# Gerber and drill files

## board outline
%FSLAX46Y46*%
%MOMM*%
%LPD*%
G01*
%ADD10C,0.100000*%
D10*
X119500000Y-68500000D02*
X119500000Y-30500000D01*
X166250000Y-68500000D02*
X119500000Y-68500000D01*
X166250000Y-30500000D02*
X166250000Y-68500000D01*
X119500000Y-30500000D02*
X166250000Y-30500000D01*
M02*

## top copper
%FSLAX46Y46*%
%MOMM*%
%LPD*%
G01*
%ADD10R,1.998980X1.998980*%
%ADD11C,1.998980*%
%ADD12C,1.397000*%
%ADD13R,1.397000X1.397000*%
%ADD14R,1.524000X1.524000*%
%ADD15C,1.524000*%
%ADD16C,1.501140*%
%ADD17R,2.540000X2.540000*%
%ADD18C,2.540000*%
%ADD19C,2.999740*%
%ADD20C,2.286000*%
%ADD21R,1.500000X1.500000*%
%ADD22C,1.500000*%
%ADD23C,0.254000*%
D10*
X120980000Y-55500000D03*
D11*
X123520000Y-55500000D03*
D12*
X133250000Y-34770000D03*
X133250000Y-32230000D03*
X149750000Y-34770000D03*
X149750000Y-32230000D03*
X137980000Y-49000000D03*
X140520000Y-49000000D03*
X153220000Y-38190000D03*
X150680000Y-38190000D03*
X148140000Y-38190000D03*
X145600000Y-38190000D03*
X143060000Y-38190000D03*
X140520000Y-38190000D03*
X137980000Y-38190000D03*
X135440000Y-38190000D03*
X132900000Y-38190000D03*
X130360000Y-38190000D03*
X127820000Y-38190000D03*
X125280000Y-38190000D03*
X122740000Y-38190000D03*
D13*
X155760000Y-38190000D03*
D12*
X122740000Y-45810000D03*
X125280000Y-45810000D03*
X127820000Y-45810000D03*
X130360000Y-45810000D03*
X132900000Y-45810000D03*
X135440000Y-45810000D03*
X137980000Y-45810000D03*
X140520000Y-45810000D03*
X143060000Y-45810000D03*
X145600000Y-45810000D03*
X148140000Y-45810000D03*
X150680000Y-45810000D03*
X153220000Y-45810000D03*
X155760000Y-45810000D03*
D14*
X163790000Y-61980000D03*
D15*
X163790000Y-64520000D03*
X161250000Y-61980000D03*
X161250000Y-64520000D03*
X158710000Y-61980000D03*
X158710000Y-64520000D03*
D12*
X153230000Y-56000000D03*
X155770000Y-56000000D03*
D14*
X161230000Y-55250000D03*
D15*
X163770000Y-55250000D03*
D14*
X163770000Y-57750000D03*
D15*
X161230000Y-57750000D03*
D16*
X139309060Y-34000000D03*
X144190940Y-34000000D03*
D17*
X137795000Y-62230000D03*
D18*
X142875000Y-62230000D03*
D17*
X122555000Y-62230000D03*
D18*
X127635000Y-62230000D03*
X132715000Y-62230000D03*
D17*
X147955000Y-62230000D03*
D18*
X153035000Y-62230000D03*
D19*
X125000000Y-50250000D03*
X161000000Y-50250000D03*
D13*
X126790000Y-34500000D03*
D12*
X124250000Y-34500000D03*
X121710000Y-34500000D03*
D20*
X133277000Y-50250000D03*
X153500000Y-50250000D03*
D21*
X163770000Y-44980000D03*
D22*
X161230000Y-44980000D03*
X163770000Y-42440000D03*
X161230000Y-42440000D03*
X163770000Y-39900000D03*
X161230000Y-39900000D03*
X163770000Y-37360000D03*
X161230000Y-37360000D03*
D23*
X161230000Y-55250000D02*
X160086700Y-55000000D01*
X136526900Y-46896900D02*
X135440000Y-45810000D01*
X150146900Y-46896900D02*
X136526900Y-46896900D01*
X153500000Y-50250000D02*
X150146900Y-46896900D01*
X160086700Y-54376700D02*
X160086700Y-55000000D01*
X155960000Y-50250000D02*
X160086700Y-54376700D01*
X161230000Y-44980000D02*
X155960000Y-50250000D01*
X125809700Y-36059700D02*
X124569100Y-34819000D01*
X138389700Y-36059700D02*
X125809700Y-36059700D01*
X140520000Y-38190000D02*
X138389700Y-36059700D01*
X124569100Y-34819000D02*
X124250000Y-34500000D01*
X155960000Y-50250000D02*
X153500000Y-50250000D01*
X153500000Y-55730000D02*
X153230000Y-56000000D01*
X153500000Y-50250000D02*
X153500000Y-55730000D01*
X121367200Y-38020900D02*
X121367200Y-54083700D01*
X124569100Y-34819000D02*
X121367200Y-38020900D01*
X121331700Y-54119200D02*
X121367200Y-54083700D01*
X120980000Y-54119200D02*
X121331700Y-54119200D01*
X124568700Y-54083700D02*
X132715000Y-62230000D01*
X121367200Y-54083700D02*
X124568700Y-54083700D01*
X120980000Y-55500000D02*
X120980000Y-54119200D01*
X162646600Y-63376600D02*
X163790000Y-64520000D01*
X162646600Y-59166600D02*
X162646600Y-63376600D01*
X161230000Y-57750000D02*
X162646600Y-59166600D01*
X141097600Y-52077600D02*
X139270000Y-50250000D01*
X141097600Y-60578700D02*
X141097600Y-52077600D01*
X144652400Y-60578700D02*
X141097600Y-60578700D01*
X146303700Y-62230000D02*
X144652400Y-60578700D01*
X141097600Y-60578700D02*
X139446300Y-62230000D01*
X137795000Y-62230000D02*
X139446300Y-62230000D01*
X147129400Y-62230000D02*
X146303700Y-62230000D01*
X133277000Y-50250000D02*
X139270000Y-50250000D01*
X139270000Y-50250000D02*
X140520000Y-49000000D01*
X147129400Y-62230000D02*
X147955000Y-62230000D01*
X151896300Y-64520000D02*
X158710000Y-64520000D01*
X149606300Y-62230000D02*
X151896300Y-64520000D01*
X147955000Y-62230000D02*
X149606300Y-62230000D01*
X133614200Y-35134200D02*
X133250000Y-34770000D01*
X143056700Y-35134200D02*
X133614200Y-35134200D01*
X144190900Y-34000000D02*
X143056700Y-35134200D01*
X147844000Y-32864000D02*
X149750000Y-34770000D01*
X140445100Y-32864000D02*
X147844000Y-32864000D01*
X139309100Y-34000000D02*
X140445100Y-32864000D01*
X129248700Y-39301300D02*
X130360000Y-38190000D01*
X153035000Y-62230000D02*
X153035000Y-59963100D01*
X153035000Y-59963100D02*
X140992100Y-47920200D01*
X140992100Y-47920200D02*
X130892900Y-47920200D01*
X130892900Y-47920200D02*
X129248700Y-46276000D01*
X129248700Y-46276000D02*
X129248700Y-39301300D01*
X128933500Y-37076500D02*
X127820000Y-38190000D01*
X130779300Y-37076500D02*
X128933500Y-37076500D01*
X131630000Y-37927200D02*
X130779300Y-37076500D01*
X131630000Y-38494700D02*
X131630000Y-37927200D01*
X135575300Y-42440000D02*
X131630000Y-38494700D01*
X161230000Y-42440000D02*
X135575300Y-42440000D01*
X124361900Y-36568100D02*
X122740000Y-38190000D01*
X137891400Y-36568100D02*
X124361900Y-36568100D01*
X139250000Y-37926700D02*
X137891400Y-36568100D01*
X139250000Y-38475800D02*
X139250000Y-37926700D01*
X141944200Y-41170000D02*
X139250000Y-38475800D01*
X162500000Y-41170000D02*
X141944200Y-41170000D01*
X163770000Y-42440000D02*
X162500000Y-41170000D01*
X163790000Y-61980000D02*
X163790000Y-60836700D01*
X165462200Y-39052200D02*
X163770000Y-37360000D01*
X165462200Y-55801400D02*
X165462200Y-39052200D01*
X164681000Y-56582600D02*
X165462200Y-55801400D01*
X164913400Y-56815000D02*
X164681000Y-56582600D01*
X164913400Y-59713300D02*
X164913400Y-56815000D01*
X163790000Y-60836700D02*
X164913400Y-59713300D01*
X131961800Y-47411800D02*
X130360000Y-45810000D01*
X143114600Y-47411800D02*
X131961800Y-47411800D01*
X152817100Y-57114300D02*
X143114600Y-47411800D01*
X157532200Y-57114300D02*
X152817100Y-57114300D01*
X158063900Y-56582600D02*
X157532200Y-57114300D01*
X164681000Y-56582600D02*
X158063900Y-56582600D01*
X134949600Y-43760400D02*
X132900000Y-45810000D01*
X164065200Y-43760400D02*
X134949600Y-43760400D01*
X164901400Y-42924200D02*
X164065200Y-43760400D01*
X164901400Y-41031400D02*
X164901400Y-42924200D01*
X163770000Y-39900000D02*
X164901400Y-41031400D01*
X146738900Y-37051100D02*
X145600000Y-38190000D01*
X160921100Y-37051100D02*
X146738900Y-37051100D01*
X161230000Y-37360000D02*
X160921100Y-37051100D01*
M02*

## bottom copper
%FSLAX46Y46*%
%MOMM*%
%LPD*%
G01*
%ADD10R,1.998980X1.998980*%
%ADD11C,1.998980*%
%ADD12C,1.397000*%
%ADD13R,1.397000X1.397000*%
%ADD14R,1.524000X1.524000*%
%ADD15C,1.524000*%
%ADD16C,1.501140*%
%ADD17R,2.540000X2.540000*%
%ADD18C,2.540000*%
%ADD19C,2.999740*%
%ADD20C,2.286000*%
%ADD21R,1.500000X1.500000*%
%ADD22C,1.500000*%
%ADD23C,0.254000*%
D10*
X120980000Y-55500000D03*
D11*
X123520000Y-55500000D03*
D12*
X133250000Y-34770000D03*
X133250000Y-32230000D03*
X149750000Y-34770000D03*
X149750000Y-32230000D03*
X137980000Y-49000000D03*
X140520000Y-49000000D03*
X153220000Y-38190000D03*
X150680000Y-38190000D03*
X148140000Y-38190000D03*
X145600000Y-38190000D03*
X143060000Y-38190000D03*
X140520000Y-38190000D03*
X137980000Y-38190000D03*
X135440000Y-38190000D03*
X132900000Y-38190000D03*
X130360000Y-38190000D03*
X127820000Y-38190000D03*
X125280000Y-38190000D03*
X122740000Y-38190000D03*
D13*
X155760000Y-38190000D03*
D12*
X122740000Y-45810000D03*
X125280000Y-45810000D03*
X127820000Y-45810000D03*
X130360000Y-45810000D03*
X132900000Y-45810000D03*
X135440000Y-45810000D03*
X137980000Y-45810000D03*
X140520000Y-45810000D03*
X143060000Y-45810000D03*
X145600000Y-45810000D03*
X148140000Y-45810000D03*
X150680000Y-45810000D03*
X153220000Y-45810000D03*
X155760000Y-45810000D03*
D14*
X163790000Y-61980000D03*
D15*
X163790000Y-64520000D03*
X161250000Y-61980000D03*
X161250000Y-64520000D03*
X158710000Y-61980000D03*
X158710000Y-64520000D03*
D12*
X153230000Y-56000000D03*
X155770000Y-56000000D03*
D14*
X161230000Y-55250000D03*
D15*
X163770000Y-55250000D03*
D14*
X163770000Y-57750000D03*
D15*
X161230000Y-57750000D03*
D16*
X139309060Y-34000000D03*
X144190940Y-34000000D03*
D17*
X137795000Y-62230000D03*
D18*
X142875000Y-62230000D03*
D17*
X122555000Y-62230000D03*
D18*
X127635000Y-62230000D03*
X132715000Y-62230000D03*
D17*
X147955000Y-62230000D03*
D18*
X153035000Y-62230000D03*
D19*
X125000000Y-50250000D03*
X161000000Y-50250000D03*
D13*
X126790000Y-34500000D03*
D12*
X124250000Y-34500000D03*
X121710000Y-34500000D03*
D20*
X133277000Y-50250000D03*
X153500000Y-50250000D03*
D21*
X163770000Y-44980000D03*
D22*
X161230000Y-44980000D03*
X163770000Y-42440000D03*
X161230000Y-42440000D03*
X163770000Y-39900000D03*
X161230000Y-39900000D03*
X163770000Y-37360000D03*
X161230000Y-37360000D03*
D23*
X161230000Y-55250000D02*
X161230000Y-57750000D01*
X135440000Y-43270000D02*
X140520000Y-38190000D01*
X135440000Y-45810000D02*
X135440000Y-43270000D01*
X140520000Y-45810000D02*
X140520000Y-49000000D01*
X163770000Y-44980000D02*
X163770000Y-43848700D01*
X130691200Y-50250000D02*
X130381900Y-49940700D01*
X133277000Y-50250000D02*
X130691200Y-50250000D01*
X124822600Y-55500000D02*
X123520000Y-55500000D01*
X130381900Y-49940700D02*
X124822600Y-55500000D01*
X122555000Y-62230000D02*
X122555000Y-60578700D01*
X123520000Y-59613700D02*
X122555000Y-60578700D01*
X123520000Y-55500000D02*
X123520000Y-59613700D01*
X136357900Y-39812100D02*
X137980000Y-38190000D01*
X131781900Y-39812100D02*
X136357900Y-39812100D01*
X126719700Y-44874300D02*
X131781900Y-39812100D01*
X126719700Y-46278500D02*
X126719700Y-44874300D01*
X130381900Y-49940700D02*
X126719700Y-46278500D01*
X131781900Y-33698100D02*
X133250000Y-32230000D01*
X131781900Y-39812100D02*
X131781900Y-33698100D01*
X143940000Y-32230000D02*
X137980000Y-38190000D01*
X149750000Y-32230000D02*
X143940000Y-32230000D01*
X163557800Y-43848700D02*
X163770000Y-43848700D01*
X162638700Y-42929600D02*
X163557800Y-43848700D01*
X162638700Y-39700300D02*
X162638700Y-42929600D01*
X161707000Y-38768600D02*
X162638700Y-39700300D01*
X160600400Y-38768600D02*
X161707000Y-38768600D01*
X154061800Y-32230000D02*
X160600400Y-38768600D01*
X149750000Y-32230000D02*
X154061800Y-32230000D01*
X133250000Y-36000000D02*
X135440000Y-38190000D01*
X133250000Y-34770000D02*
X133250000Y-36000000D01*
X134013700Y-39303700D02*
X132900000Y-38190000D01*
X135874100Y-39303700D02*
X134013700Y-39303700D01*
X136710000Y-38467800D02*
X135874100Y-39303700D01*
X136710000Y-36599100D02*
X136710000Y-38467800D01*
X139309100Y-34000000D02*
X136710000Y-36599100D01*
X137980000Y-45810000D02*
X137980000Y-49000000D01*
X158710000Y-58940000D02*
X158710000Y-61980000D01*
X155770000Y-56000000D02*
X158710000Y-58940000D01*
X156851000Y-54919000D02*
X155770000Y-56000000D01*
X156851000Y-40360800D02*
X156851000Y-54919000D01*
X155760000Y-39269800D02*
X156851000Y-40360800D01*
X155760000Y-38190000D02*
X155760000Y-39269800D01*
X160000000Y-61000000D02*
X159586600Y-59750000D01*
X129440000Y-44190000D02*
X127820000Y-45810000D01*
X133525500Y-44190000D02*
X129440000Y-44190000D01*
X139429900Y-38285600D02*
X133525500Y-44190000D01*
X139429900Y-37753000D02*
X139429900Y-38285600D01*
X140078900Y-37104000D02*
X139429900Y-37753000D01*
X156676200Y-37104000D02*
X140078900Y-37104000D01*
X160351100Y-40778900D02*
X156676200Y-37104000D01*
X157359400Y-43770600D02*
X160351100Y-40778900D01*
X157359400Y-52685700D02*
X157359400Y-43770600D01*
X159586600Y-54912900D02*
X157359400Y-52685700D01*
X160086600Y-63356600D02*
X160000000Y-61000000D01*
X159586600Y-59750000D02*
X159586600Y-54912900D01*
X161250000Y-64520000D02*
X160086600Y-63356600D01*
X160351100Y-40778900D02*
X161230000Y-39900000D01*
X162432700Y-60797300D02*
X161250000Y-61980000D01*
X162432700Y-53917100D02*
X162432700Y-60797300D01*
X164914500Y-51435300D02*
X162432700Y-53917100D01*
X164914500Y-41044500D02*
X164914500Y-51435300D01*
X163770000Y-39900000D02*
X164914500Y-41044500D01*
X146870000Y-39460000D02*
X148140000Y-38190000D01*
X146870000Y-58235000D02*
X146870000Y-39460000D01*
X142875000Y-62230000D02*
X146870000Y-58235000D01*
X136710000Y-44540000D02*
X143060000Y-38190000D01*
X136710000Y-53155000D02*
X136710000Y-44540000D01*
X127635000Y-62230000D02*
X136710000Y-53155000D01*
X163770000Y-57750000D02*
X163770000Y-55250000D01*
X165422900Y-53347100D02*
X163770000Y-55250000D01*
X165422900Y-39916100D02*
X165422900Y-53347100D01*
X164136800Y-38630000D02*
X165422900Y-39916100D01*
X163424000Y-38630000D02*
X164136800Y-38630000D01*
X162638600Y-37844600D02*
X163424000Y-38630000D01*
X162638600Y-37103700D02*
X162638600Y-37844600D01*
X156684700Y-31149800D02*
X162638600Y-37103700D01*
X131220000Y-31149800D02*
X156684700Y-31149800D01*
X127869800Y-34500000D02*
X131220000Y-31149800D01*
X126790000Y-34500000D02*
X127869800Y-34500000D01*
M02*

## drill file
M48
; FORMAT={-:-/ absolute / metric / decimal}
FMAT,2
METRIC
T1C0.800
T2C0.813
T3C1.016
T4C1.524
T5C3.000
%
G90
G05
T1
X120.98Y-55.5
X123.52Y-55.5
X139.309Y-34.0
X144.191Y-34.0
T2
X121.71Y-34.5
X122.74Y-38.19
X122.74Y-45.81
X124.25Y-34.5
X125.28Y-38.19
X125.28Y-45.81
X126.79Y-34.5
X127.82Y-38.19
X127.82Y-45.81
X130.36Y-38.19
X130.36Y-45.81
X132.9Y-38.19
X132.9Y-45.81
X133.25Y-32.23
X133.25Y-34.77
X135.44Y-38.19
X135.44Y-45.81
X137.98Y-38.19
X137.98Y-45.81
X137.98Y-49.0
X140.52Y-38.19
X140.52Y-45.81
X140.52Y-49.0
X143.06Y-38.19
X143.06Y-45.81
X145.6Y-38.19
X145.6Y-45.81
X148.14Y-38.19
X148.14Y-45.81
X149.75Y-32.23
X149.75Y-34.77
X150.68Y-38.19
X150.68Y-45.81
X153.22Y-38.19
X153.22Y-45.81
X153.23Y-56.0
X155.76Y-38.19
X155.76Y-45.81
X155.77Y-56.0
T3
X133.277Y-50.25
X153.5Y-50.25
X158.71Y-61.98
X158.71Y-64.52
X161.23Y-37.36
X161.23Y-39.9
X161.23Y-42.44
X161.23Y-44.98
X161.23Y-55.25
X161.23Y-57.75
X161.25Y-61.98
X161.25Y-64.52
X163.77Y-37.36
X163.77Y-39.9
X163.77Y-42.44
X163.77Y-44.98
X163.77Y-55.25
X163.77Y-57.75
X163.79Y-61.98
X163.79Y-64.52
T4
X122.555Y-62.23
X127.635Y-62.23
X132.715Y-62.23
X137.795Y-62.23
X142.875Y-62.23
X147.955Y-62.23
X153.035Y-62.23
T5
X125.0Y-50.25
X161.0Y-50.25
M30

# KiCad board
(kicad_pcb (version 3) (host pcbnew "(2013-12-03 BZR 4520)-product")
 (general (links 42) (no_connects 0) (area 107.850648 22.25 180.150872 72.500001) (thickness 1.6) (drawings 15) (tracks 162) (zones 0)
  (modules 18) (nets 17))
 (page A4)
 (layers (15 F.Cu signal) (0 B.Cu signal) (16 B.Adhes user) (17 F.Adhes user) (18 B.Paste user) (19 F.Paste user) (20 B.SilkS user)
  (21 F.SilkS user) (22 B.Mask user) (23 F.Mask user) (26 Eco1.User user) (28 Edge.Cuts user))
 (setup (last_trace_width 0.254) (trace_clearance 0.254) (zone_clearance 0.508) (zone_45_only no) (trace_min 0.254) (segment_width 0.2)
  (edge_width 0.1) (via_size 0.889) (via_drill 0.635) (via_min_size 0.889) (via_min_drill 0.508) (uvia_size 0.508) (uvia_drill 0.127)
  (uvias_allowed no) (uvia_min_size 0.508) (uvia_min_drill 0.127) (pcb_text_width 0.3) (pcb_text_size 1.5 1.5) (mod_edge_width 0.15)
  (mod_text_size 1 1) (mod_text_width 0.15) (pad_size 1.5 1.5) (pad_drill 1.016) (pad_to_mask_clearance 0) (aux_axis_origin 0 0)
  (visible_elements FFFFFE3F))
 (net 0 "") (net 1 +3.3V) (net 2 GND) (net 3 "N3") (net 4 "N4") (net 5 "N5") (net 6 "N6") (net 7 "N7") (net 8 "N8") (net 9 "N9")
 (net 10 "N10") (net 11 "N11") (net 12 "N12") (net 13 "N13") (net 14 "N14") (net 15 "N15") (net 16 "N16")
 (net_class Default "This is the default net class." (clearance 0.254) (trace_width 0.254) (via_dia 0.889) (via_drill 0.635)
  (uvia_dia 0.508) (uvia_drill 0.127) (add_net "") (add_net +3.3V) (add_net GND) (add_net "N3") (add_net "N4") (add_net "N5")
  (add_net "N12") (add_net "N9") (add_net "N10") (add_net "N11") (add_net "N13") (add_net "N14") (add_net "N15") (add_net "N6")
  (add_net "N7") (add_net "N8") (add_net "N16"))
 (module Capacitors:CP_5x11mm (layer F.Cu) (at 122.25 55.5 270)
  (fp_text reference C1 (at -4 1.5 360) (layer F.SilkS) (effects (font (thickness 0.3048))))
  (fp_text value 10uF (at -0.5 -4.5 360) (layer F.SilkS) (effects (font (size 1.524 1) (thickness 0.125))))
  (pad 1 thru_hole rect (at 0 1.27 270) (size 1.99898 1.99898) (drill 0.8001) (layers *.Cu *.Mask F.SilkS) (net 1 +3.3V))
  (pad 2 thru_hole circle (at 0 -1.27 270) (size 1.99898 1.99898) (drill 0.8001) (layers *.Cu *.Mask F.SilkS) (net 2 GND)))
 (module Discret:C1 (layer F.Cu) (at 133.25 33.5 90)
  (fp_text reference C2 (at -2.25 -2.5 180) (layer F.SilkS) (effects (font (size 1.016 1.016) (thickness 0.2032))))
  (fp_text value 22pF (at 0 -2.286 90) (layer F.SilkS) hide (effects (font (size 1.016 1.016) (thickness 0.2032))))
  (pad 1 thru_hole circle (at -1.27 0 90) (size 1.397 1.397) (drill 0.8128) (layers *.Cu *.Mask F.SilkS) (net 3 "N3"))
  (pad 2 thru_hole circle (at 1.27 0 90) (size 1.397 1.397) (drill 0.8128) (layers *.Cu *.Mask F.SilkS) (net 2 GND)))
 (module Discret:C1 (layer F.Cu) (at 149.75 33.5 90)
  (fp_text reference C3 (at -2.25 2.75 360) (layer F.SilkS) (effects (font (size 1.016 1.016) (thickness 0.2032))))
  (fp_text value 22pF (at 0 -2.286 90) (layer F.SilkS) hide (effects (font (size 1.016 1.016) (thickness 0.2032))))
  (pad 1 thru_hole circle (at -1.27 0 90) (size 1.397 1.397) (drill 0.8128) (layers *.Cu *.Mask F.SilkS) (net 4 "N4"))
  (pad 2 thru_hole circle (at 1.27 0 90) (size 1.397 1.397) (drill 0.8128) (layers *.Cu *.Mask F.SilkS) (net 2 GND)))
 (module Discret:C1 (layer F.Cu) (at 139.25 49)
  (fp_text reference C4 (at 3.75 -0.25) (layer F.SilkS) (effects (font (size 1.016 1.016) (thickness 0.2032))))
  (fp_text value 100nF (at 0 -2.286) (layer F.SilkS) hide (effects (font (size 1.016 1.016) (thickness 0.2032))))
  (pad 1 thru_hole circle (at -1.27 0) (size 1.397 1.397) (drill 0.8128) (layers *.Cu *.Mask F.SilkS) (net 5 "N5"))
  (pad 2 thru_hole circle (at 1.27 0) (size 1.397 1.397) (drill 0.8128) (layers *.Cu *.Mask F.SilkS) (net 2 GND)))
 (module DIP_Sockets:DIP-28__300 (layer F.Cu) (at 139.25 42 180)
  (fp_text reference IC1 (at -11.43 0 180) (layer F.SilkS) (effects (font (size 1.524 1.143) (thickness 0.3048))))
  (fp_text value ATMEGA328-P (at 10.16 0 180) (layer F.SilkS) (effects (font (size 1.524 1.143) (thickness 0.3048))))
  (pad 2 thru_hole circle (at -13.97 3.81 180) (size 1.397 1.397) (drill 0.8128) (layers *.Cu *.Mask F.SilkS))
  (pad 3 thru_hole circle (at -11.43 3.81 180) (size 1.397 1.397) (drill 0.8128) (layers *.Cu *.Mask F.SilkS))
  (pad 4 thru_hole circle (at -8.89 3.81 180) (size 1.397 1.397) (drill 0.8128) (layers *.Cu *.Mask F.SilkS) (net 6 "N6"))
  (pad 5 thru_hole circle (at -6.35 3.81 180) (size 1.397 1.397) (drill 0.8128) (layers *.Cu *.Mask F.SilkS) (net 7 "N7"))
  (pad 6 thru_hole circle (at -3.81 3.81 180) (size 1.397 1.397) (drill 0.8128) (layers *.Cu *.Mask F.SilkS) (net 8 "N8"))
  (pad 7 thru_hole circle (at -1.27 3.81 180) (size 1.397 1.397) (drill 0.8128) (layers *.Cu *.Mask F.SilkS) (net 1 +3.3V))
  (pad 8 thru_hole circle (at 1.27 3.81 180) (size 1.397 1.397) (drill 0.8128) (layers *.Cu *.Mask F.SilkS) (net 2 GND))
  (pad 9 thru_hole circle (at 3.81 3.81 180) (size 1.397 1.397) (drill 0.8128) (layers *.Cu *.Mask F.SilkS) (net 3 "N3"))
  (pad 10 thru_hole circle (at 6.35 3.81 180) (size 1.397 1.397) (drill 0.8128) (layers *.Cu *.Mask F.SilkS) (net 4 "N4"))
  (pad 11 thru_hole circle (at 8.89 3.81 180) (size 1.397 1.397) (drill 0.8128) (layers *.Cu *.Mask F.SilkS) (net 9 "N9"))
  (pad 12 thru_hole circle (at 11.43 3.81 180) (size 1.397 1.397) (drill 0.8128) (layers *.Cu *.Mask F.SilkS) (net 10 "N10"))
  (pad 13 thru_hole circle (at 13.97 3.81 180) (size 1.397 1.397) (drill 0.8128) (layers *.Cu *.Mask F.SilkS))
  (pad 14 thru_hole circle (at 16.51 3.81 180) (size 1.397 1.397) (drill 0.8128) (layers *.Cu *.Mask F.SilkS) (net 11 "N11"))
  (pad 1 thru_hole rect (at -16.51 3.81 180) (size 1.397 1.397) (drill 0.8128) (layers *.Cu *.Mask F.SilkS) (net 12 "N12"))
  (pad 15 thru_hole circle (at 16.51 -3.81 180) (size 1.397 1.397) (drill 0.8128) (layers *.Cu *.Mask F.SilkS))
  (pad 16 thru_hole circle (at 13.97 -3.81 180) (size 1.397 1.397) (drill 0.8128) (layers *.Cu *.Mask F.SilkS))
  (pad 17 thru_hole circle (at 11.43 -3.81 180) (size 1.397 1.397) (drill 0.8128) (layers *.Cu *.Mask F.SilkS) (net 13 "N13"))
  (pad 18 thru_hole circle (at 8.89 -3.81 180) (size 1.397 1.397) (drill 0.8128) (layers *.Cu *.Mask F.SilkS) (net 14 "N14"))
  (pad 19 thru_hole circle (at 6.35 -3.81 180) (size 1.397 1.397) (drill 0.8128) (layers *.Cu *.Mask F.SilkS) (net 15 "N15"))
  (pad 20 thru_hole circle (at 3.81 -3.81 180) (size 1.397 1.397) (drill 0.8128) (layers *.Cu *.Mask F.SilkS) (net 1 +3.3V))
  (pad 21 thru_hole circle (at 1.27 -3.81 180) (size 1.397 1.397) (drill 0.8128) (layers *.Cu *.Mask F.SilkS) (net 5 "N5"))
  (pad 22 thru_hole circle (at -1.27 -3.81 180) (size 1.397 1.397) (drill 0.8128) (layers *.Cu *.Mask F.SilkS) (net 2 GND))
  (pad 23 thru_hole circle (at -3.81 -3.81 180) (size 1.397 1.397) (drill 0.8128) (layers *.Cu *.Mask F.SilkS))
  (pad 24 thru_hole circle (at -6.35 -3.81 180) (size 1.397 1.397) (drill 0.8128) (layers *.Cu *.Mask F.SilkS))
  (pad 25 thru_hole circle (at -8.89 -3.81 180) (size 1.397 1.397) (drill 0.8128) (layers *.Cu *.Mask F.SilkS))
  (pad 26 thru_hole circle (at -11.43 -3.81 180) (size 1.397 1.397) (drill 0.8128) (layers *.Cu *.Mask F.SilkS))
  (pad 27 thru_hole circle (at -13.97 -3.81 180) (size 1.397 1.397) (drill 0.8128) (layers *.Cu *.Mask F.SilkS))
  (pad 28 thru_hole circle (at -16.51 -3.81 180) (size 1.397 1.397) (drill 0.8128) (layers *.Cu *.Mask F.SilkS)))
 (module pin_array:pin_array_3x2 (layer F.Cu) (at 161.25 63.25 180)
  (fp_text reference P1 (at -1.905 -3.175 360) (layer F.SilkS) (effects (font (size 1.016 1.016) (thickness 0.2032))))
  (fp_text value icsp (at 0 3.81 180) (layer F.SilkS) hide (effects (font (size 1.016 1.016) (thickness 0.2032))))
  (pad 1 thru_hole rect (at -2.54 1.27 180) (size 1.524 1.524) (drill 1.016) (layers *.Cu *.Mask F.SilkS) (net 14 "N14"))
  (pad 2 thru_hole circle (at -2.54 -1.27 180) (size 1.524 1.524) (drill 1.016) (layers *.Cu *.Mask F.SilkS) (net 1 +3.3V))
  (pad 3 thru_hole circle (at 0 1.27 180) (size 1.524 1.524) (drill 1.016) (layers *.Cu *.Mask F.SilkS) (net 15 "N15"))
  (pad 4 thru_hole circle (at 0 -1.27 180) (size 1.524 1.524) (drill 1.016) (layers *.Cu *.Mask F.SilkS) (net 13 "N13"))
  (pad 5 thru_hole circle (at 2.54 1.27 180) (size 1.524 1.524) (drill 1.016) (layers *.Cu *.Mask F.SilkS) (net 12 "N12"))
  (pad 6 thru_hole circle (at 2.54 -1.27 180) (size 1.524 1.524) (drill 1.016) (layers *.Cu *.Mask F.SilkS) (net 2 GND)))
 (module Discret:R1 (layer F.Cu) (at 154.5 56) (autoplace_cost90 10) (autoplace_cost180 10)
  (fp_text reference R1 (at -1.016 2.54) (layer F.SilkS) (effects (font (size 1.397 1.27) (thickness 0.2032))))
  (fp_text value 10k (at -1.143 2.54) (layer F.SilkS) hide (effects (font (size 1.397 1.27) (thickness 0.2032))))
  (pad 1 thru_hole circle (at -1.27 0) (size 1.397 1.397) (drill 0.8128) (layers *.Cu *.Mask F.SilkS) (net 1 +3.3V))
  (pad 2 thru_hole circle (at 1.27 0) (size 1.397 1.397) (drill 0.8128) (layers *.Cu *.Mask F.SilkS) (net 12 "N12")))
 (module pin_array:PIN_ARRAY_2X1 (layer F.Cu) (at 162.5 55.25)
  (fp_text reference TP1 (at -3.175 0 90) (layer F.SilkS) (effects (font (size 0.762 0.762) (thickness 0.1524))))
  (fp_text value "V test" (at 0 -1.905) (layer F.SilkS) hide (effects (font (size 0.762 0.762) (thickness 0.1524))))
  (pad 1 thru_hole rect (at -1.27 0) (size 1.524 1.524) (drill 1.016) (layers *.Cu *.Mask F.SilkS) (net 1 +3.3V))
  (pad 2 thru_hole circle (at 1.27 0) (size 1.524 1.524) (drill 1.016) (layers *.Cu *.Mask F.SilkS) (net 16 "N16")))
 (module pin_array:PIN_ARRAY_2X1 (layer F.Cu) (at 162.5 57.75 180)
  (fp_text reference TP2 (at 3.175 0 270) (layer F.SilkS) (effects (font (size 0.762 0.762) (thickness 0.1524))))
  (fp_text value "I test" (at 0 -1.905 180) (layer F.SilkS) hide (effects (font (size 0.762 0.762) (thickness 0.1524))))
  (pad 1 thru_hole rect (at -1.27 0 180) (size 1.524 1.524) (drill 1.016) (layers *.Cu *.Mask F.SilkS) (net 16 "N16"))
  (pad 2 thru_hole circle (at 1.27 0 180) (size 1.524 1.524) (drill 1.016) (layers *.Cu *.Mask F.SilkS) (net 1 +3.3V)))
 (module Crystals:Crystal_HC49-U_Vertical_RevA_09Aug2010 (layer F.Cu) (at 141.75 34)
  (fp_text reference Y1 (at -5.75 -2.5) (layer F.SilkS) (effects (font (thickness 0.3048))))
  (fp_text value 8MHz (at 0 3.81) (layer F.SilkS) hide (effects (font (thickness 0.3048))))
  (pad 1 thru_hole circle (at -2.44094 0) (size 1.50114 1.50114) (drill 0.8001) (layers *.Cu *.Mask F.SilkS) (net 4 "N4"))
  (pad 2 thru_hole circle (at 2.44094 0) (size 1.50114 1.50114) (drill 0.8001) (layers *.Cu *.Mask F.SilkS) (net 3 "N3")))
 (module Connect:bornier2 (layer F.Cu) (at 140.335 62.23)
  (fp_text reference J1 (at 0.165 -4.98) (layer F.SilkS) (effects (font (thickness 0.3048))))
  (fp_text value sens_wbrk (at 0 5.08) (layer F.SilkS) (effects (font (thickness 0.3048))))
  (pad 1 thru_hole rect (at -2.54 0) (size 2.54 2.54) (drill 1.524) (layers *.Cu *.Mask F.SilkS) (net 2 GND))
  (pad 2 thru_hole circle (at 2.54 0) (size 2.54 2.54) (drill 1.524) (layers *.Cu *.Mask F.SilkS) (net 6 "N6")))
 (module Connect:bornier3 (layer F.Cu) (at 127.635 62.23)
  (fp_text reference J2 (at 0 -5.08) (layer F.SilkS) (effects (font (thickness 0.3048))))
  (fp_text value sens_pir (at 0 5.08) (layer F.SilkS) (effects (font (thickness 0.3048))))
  (pad 1 thru_hole rect (at -5.08 0) (size 2.54 2.54) (drill 1.524) (layers *.Cu *.Mask F.SilkS) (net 2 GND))
  (pad 2 thru_hole circle (at 0 0) (size 2.54 2.54) (drill 1.524) (layers *.Cu *.Mask F.SilkS) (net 8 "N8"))
  (pad 3 thru_hole circle (at 5.08 0) (size 2.54 2.54) (drill 1.524) (layers *.Cu *.Mask F.SilkS) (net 1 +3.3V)))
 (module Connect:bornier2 (layer F.Cu) (at 150.495 62.23)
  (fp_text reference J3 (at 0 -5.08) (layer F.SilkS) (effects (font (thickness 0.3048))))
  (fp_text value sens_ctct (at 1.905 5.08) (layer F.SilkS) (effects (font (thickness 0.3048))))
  (pad 1 thru_hole rect (at -2.54 0) (size 2.54 2.54) (drill 1.524) (layers *.Cu *.Mask F.SilkS) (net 2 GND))
  (pad 2 thru_hole circle (at 2.54 0) (size 2.54 2.54) (drill 1.524) (layers *.Cu *.Mask F.SilkS) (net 9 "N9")))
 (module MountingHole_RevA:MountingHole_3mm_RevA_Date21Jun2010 (layer F.Cu) (at 125 50.25) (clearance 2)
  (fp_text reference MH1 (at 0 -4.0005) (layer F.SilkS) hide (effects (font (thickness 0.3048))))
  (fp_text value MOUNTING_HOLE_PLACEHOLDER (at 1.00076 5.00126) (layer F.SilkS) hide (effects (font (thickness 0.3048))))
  (pad 1 thru_hole circle (at 0 0) (size 2.99974 2.99974) (drill 2.99974) (layers)))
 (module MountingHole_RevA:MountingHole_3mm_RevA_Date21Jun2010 (layer F.Cu) (at 161 50.25) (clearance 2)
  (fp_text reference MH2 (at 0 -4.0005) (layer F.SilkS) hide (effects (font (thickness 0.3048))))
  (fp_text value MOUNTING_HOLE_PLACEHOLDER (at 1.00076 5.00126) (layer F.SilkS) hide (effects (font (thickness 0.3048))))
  (pad 1 thru_hole circle (at 0 0) (size 2.99974 2.99974) (drill 2.99974) (layers)))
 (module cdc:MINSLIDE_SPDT (layer F.Cu) (at 124.25 34.5 180)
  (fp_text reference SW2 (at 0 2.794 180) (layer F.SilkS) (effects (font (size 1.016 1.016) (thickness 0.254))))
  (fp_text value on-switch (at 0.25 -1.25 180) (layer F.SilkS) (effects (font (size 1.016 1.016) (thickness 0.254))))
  (pad 1 thru_hole rect (at -2.54 0 180) (size 1.397 1.397) (drill 0.8128) (layers *.Cu *.Mask F.SilkS) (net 16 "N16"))
  (pad 2 thru_hole circle (at 0 0 180) (size 1.397 1.397) (drill 0.8128) (layers *.Cu *.Mask F.SilkS) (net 1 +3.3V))
  (pad 3 thru_hole circle (at 2.54 0 180) (size 1.397 1.397) (drill 0.8128) (layers *.Cu *.Mask F.SilkS)))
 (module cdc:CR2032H (layer B.Cu) (at 139.5 50.25)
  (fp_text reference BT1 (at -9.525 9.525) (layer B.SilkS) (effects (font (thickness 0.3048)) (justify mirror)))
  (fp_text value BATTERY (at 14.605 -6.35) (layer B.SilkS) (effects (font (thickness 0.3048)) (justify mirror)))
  (pad 2 thru_hole circle (at -6.223 0) (size 2.286 2.286) (drill 1.016) (layers *.Cu *.Mask B.SilkS) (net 2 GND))
  (pad 1 thru_hole circle (at 14 0) (size 2.286 2.286) (drill 1.016) (layers *.Cu *.Mask B.SilkS) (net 1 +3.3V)))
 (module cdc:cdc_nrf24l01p (layer F.Cu) (at 162.5 46.25 180)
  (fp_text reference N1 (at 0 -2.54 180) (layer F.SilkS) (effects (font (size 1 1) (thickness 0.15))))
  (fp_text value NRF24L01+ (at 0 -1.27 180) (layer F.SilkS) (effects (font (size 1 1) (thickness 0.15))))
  (pad 1 thru_hole rect (at -1.27 1.27 180) (size 1.5 1.5) (drill 1.016) (layers *.Cu *.Mask F.SilkS) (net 2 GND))
  (pad 2 thru_hole circle (at 1.27 1.27 180) (size 1.5 1.5) (drill 1.016) (layers *.Cu *.Mask F.SilkS) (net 1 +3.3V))
  (pad 3 thru_hole circle (at -1.27 3.81 180) (size 1.5 1.5) (drill 1.016) (layers *.Cu *.Mask F.SilkS) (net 11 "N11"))
  (pad 4 thru_hole circle (at 1.27 3.81 180) (size 1.5 1.5) (drill 1.016) (layers *.Cu *.Mask F.SilkS) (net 10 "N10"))
  (pad 5 thru_hole circle (at -1.27 6.35 180) (size 1.5 1.5) (drill 1.016) (layers *.Cu *.Mask F.SilkS) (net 15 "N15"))
  (pad 6 thru_hole circle (at 1.27 6.35 180) (size 1.5 1.5) (drill 1.016) (layers *.Cu *.Mask F.SilkS) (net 13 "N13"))
  (pad 7 thru_hole circle (at -1.27 8.89 180) (size 1.5 1.5) (drill 1.016) (layers *.Cu *.Mask F.SilkS) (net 14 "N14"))
  (pad 8 thru_hole circle (at 1.27 8.89 180) (size 1.5 1.5) (drill 1.016) (layers *.Cu *.Mask F.SilkS) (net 7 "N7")))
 (gr_line (start 119.5 68.5) (end 119.5 30.5) (angle 90) (layer Edge.Cuts) (width 0.1))
 (gr_line (start 166.25 68.5) (end 119.5 68.5) (angle 90) (layer Edge.Cuts) (width 0.1))
 (gr_line (start 166.25 30.5) (end 166.25 68.5) (angle 90) (layer Edge.Cuts) (width 0.1))
 (gr_line (start 119.5 30.5) (end 166.25 30.5) (angle 90) (layer Edge.Cuts) (width 0.1))
 (segment (start 161.23 55.25) (end 161.23 57.75) (width 0.254) (layer B.Cu) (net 1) (status 20))
 (segment (start 161.23 55.25) (end 160.0867 55) (width 0.254) (layer F.Cu) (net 1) (status 10))
 (segment (start 136.5269 46.8969) (end 135.44 45.81) (width 0.254) (layer F.Cu) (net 1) (status 20))
 (segment (start 150.1469 46.8969) (end 136.5269 46.8969) (width 0.254) (layer F.Cu) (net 1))
 (segment (start 153.5 50.25) (end 150.1469 46.8969) (width 0.254) (layer F.Cu) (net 1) (status 10))
 (segment (start 160.0867 54.3767) (end 160.0867 55) (width 0.254) (layer F.Cu) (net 1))
 (segment (start 155.96 50.25) (end 160.0867 54.3767) (width 0.254) (layer F.Cu) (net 1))
 (segment (start 161.23 44.98) (end 155.96 50.25) (width 0.254) (layer F.Cu) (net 1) (status 10))
 (segment (start 135.44 43.27) (end 140.52 38.19) (width 0.254) (layer B.Cu) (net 1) (status 20))
 (segment (start 135.44 45.81) (end 135.44 43.27) (width 0.254) (layer B.Cu) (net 1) (status 10))
 (segment (start 125.8097 36.0597) (end 124.5691 34.819) (width 0.254) (layer F.Cu) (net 1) (status 20))
 (segment (start 138.3897 36.0597) (end 125.8097 36.0597) (width 0.254) (layer F.Cu) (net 1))
 (segment (start 140.52 38.19) (end 138.3897 36.0597) (width 0.254) (layer F.Cu) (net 1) (status 10))
 (segment (start 124.5691 34.819) (end 124.25 34.5) (width 0.254) (layer F.Cu) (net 1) (status 30))
 (segment (start 155.96 50.25) (end 153.5 50.25) (width 0.254) (layer F.Cu) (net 1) (status 20))
 (segment (start 153.5 55.73) (end 153.23 56) (width 0.254) (layer F.Cu) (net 1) (status 30))
 (segment (start 153.5 50.25) (end 153.5 55.73) (width 0.254) (layer F.Cu) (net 1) (status 30))
 (segment (start 121.3672 38.0209) (end 121.3672 54.0837) (width 0.254) (layer F.Cu) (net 1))
 (segment (start 124.5691 34.819) (end 121.3672 38.0209) (width 0.254) (layer F.Cu) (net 1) (status 10))
 (segment (start 121.3317 54.1192) (end 121.3672 54.0837) (width 0.254) (layer F.Cu) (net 1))
 (segment (start 120.98 54.1192) (end 121.3317 54.1192) (width 0.254) (layer F.Cu) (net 1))
 (segment (start 124.5687 54.0837) (end 132.715 62.23) (width 0.254) (layer F.Cu) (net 1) (status 20))
 (segment (start 121.3672 54.0837) (end 124.5687 54.0837) (width 0.254) (layer F.Cu) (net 1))
 (segment (start 120.98 55.5) (end 120.98 54.1192) (width 0.254) (layer F.Cu) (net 1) (status 10))
 (segment (start 162.6466 63.3766) (end 163.79 64.52) (width 0.254) (layer F.Cu) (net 1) (status 20))
 (segment (start 162.6466 59.1666) (end 162.6466 63.3766) (width 0.254) (layer F.Cu) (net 1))
 (segment (start 161.23 57.75) (end 162.6466 59.1666) (width 0.254) (layer F.Cu) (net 1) (status 10))
 (segment (start 141.0976 52.0776) (end 139.27 50.25) (width 0.254) (layer F.Cu) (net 2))
 (segment (start 141.0976 60.5787) (end 141.0976 52.0776) (width 0.254) (layer F.Cu) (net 2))
 (segment (start 144.6524 60.5787) (end 141.0976 60.5787) (width 0.254) (layer F.Cu) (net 2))
 (segment (start 146.3037 62.23) (end 144.6524 60.5787) (width 0.254) (layer F.Cu) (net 2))
 (segment (start 141.0976 60.5787) (end 139.4463 62.23) (width 0.254) (layer F.Cu) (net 2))
 (segment (start 140.52 45.81) (end 140.52 49) (width 0.254) (layer B.Cu) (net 2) (status 30))
 (segment (start 163.77 44.98) (end 163.77 43.8487) (width 0.254) (layer B.Cu) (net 2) (status 10))
 (segment (start 137.795 62.23) (end 139.4463 62.23) (width 0.254) (layer F.Cu) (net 2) (status 10))
 (segment (start 147.1294 62.23) (end 146.3037 62.23) (width 0.254) (layer F.Cu) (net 2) (status 10))
 (segment (start 133.277 50.25) (end 139.27 50.25) (width 0.254) (layer F.Cu) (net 2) (status 10))
 (segment (start 139.27 50.25) (end 140.52 49) (width 0.254) (layer F.Cu) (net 2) (status 20))
 (segment (start 130.6912 50.25) (end 130.3819 49.9407) (width 0.254) (layer B.Cu) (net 2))
 (segment (start 133.277 50.25) (end 130.6912 50.25) (width 0.254) (layer B.Cu) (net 2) (status 10))
 (segment (start 147.1294 62.23) (end 147.955 62.23) (width 0.254) (layer F.Cu) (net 2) (status 30))
 (segment (start 151.8963 64.52) (end 158.71 64.52) (width 0.254) (layer F.Cu) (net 2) (status 20))
 (segment (start 149.6063 62.23) (end 151.8963 64.52) (width 0.254) (layer F.Cu) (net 2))
 (segment (start 147.955 62.23) (end 149.6063 62.23) (width 0.254) (layer F.Cu) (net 2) (status 10))
 (segment (start 124.8226 55.5) (end 123.52 55.5) (width 0.254) (layer B.Cu) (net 2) (status 20))
 (segment (start 130.3819 49.9407) (end 124.8226 55.5) (width 0.254) (layer B.Cu) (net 2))
 (segment (start 122.555 62.23) (end 122.555 60.5787) (width 0.254) (layer B.Cu) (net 2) (status 10))
 (segment (start 123.52 59.6137) (end 122.555 60.5787) (width 0.254) (layer B.Cu) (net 2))
 (segment (start 123.52 55.5) (end 123.52 59.6137) (width 0.254) (layer B.Cu) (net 2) (status 10))
 (segment (start 136.3579 39.8121) (end 137.98 38.19) (width 0.254) (layer B.Cu) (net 2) (status 20))
 (segment (start 131.7819 39.8121) (end 136.3579 39.8121) (width 0.254) (layer B.Cu) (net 2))
 (segment (start 126.7197 44.8743) (end 131.7819 39.8121) (width 0.254) (layer B.Cu) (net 2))
 (segment (start 126.7197 46.2785) (end 126.7197 44.8743) (width 0.254) (layer B.Cu) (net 2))
 (segment (start 130.3819 49.9407) (end 126.7197 46.2785) (width 0.254) (layer B.Cu) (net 2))
 (segment (start 131.7819 33.6981) (end 133.25 32.23) (width 0.254) (layer B.Cu) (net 2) (status 20))
 (segment (start 131.7819 39.8121) (end 131.7819 33.6981) (width 0.254) (layer B.Cu) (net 2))
 (segment (start 143.94 32.23) (end 137.98 38.19) (width 0.254) (layer B.Cu) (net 2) (status 20))
 (segment (start 149.75 32.23) (end 143.94 32.23) (width 0.254) (layer B.Cu) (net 2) (status 10))
 (segment (start 163.5578 43.8487) (end 163.77 43.8487) (width 0.254) (layer B.Cu) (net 2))
 (segment (start 162.6387 42.9296) (end 163.5578 43.8487) (width 0.254) (layer B.Cu) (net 2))
 (segment (start 162.6387 39.7003) (end 162.6387 42.9296) (width 0.254) (layer B.Cu) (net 2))
 (segment (start 161.707 38.7686) (end 162.6387 39.7003) (width 0.254) (layer B.Cu) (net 2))
 (segment (start 160.6004 38.7686) (end 161.707 38.7686) (width 0.254) (layer B.Cu) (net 2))
 (segment (start 154.0618 32.23) (end 160.6004 38.7686) (width 0.254) (layer B.Cu) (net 2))
 (segment (start 149.75 32.23) (end 154.0618 32.23) (width 0.254) (layer B.Cu) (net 2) (status 10))
 (segment (start 133.6142 35.1342) (end 133.25 34.77) (width 0.254) (layer F.Cu) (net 3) (status 30))
 (segment (start 143.0567 35.1342) (end 133.6142 35.1342) (width 0.254) (layer F.Cu) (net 3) (status 20))
 (segment (start 144.1909 34) (end 143.0567 35.1342) (width 0.254) (layer F.Cu) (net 3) (status 10))
 (segment (start 133.25 36) (end 135.44 38.19) (width 0.254) (layer B.Cu) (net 3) (status 20))
 (segment (start 133.25 34.77) (end 133.25 36) (width 0.254) (layer B.Cu) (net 3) (status 10))
 (segment (start 147.844 32.864) (end 149.75 34.77) (width 0.254) (layer F.Cu) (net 4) (status 20))
 (segment (start 140.4451 32.864) (end 147.844 32.864) (width 0.254) (layer F.Cu) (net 4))
 (segment (start 139.3091 34) (end 140.4451 32.864) (width 0.254) (layer F.Cu) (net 4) (status 10))
 (segment (start 134.0137 39.3037) (end 132.9 38.19) (width 0.254) (layer B.Cu) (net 4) (status 20))
 (segment (start 135.8741 39.3037) (end 134.0137 39.3037) (width 0.254) (layer B.Cu) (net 4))
 (segment (start 136.71 38.4678) (end 135.8741 39.3037) (width 0.254) (layer B.Cu) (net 4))
 (segment (start 136.71 36.5991) (end 136.71 38.4678) (width 0.254) (layer B.Cu) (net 4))
 (segment (start 139.3091 34) (end 136.71 36.5991) (width 0.254) (layer B.Cu) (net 4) (status 10))
 (segment (start 137.98 45.81) (end 137.98 49) (width 0.254) (layer B.Cu) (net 5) (status 30))
 (segment (start 158.71 58.94) (end 158.71 61.98) (width 0.254) (layer B.Cu) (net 12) (status 20))
 (segment (start 155.77 56) (end 158.71 58.94) (width 0.254) (layer B.Cu) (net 12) (status 10))
 (segment (start 156.851 54.919) (end 155.77 56) (width 0.254) (layer B.Cu) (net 12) (status 20))
 (segment (start 156.851 40.3608) (end 156.851 54.919) (width 0.254) (layer B.Cu) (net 12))
 (segment (start 155.76 39.2698) (end 156.851 40.3608) (width 0.254) (layer B.Cu) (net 12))
 (segment (start 155.76 38.19) (end 155.76 39.2698) (width 0.254) (layer B.Cu) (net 12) (status 10))
 (segment (start 129.2487 39.3013) (end 130.36 38.19) (width 0.254) (layer F.Cu) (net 9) (status 20))
 (segment (start 153.035 62.23) (end 153.035 59.9631) (width 0.254) (layer F.Cu) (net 9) (status 10))
 (segment (start 153.035 59.9631) (end 140.9921 47.9202) (width 0.254) (layer F.Cu) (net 9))
 (segment (start 140.9921 47.9202) (end 130.8929 47.9202) (width 0.254) (layer F.Cu) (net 9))
 (segment (start 130.8929 47.9202) (end 129.2487 46.276) (width 0.254) (layer F.Cu) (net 9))
 (segment (start 129.2487 46.276) (end 129.2487 39.3013) (width 0.254) (layer F.Cu) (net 9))
 (segment (start 128.9335 37.0765) (end 127.82 38.19) (width 0.254) (layer F.Cu) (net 10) (status 20))
 (segment (start 130.7793 37.0765) (end 128.9335 37.0765) (width 0.254) (layer F.Cu) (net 10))
 (segment (start 131.63 37.9272) (end 130.7793 37.0765) (width 0.254) (layer F.Cu) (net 10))
 (segment (start 131.63 38.4947) (end 131.63 37.9272) (width 0.254) (layer F.Cu) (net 10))
 (segment (start 135.5753 42.44) (end 131.63 38.4947) (width 0.254) (layer F.Cu) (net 10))
 (segment (start 161.23 42.44) (end 135.5753 42.44) (width 0.254) (layer F.Cu) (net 10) (status 10))
 (segment (start 124.3619 36.5681) (end 122.74 38.19) (width 0.254) (layer F.Cu) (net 11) (status 20))
 (segment (start 137.8914 36.5681) (end 124.3619 36.5681) (width 0.254) (layer F.Cu) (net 11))
 (segment (start 139.25 37.9267) (end 137.8914 36.5681) (width 0.254) (layer F.Cu) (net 11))
 (segment (start 139.25 38.4758) (end 139.25 37.9267) (width 0.254) (layer F.Cu) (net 11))
 (segment (start 141.9442 41.17) (end 139.25 38.4758) (width 0.254) (layer F.Cu) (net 11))
 (segment (start 162.5 41.17) (end 141.9442 41.17) (width 0.254) (layer F.Cu) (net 11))
 (segment (start 163.77 42.44) (end 162.5 41.17) (width 0.254) (layer F.Cu) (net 11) (status 10))
 (segment (start 160 61) (end 159.5866 59.75) (width 0.254) (layer B.Cu) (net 13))
 (segment (start 129.44 44.19) (end 127.82 45.81) (width 0.254) (layer B.Cu) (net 13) (status 20))
 (segment (start 133.5255 44.19) (end 129.44 44.19) (width 0.254) (layer B.Cu) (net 13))
 (segment (start 139.4299 38.2856) (end 133.5255 44.19) (width 0.254) (layer B.Cu) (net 13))
 (segment (start 139.4299 37.753) (end 139.4299 38.2856) (width 0.254) (layer B.Cu) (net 13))
 (segment (start 140.0789 37.104) (end 139.4299 37.753) (width 0.254) (layer B.Cu) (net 13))
 (segment (start 156.6762 37.104) (end 140.0789 37.104) (width 0.254) (layer B.Cu) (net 13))
 (segment (start 160.3511 40.7789) (end 156.6762 37.104) (width 0.254) (layer B.Cu) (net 13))
 (segment (start 157.3594 43.7706) (end 160.3511 40.7789) (width 0.254) (layer B.Cu) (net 13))
 (segment (start 157.3594 52.6857) (end 157.3594 43.7706) (width 0.254) (layer B.Cu) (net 13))
 (segment (start 159.5866 54.9129) (end 157.3594 52.6857) (width 0.254) (layer B.Cu) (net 13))
 (segment (start 160.0866 63.3566) (end 160 61) (width 0.254) (layer B.Cu) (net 13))
 (segment (start 159.5866 59.75) (end 159.5866 54.9129) (width 0.254) (layer B.Cu) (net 13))
 (segment (start 161.25 64.52) (end 160.0866 63.3566) (width 0.254) (layer B.Cu) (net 13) (status 10))
 (segment (start 160.3511 40.7789) (end 161.23 39.9) (width 0.254) (layer B.Cu) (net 13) (status 20))
 (segment (start 163.79 61.98) (end 163.79 60.8367) (width 0.254) (layer F.Cu) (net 14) (status 10))
 (segment (start 165.4622 39.0522) (end 163.77 37.36) (width 0.254) (layer F.Cu) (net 14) (status 20))
 (segment (start 165.4622 55.8014) (end 165.4622 39.0522) (width 0.254) (layer F.Cu) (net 14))
 (segment (start 164.681 56.5826) (end 165.4622 55.8014) (width 0.254) (layer F.Cu) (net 14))
 (segment (start 164.9134 56.815) (end 164.681 56.5826) (width 0.254) (layer F.Cu) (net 14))
 (segment (start 164.9134 59.7133) (end 164.9134 56.815) (width 0.254) (layer F.Cu) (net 14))
 (segment (start 163.79 60.8367) (end 164.9134 59.7133) (width 0.254) (layer F.Cu) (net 14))
 (segment (start 131.9618 47.4118) (end 130.36 45.81) (width 0.254) (layer F.Cu) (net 14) (status 20))
 (segment (start 143.1146 47.4118) (end 131.9618 47.4118) (width 0.254) (layer F.Cu) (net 14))
 (segment (start 152.8171 57.1143) (end 143.1146 47.4118) (width 0.254) (layer F.Cu) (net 14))
 (segment (start 157.5322 57.1143) (end 152.8171 57.1143) (width 0.254) (layer F.Cu) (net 14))
 (segment (start 158.0639 56.5826) (end 157.5322 57.1143) (width 0.254) (layer F.Cu) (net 14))
 (segment (start 164.681 56.5826) (end 158.0639 56.5826) (width 0.254) (layer F.Cu) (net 14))
 (segment (start 134.9496 43.7604) (end 132.9 45.81) (width 0.254) (layer F.Cu) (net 15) (status 20))
 (segment (start 164.0652 43.7604) (end 134.9496 43.7604) (width 0.254) (layer F.Cu) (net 15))
 (segment (start 164.9014 42.9242) (end 164.0652 43.7604) (width 0.254) (layer F.Cu) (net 15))
 (segment (start 164.9014 41.0314) (end 164.9014 42.9242) (width 0.254) (layer F.Cu) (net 15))
 (segment (start 163.77 39.9) (end 164.9014 41.0314) (width 0.254) (layer F.Cu) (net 15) (status 10))
 (segment (start 162.4327 60.7973) (end 161.25 61.98) (width 0.254) (layer B.Cu) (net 15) (status 20))
 (segment (start 162.4327 53.9171) (end 162.4327 60.7973) (width 0.254) (layer B.Cu) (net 15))
 (segment (start 164.9145 51.4353) (end 162.4327 53.9171) (width 0.254) (layer B.Cu) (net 15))
 (segment (start 164.9145 41.0445) (end 164.9145 51.4353) (width 0.254) (layer B.Cu) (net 15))
 (segment (start 163.77 39.9) (end 164.9145 41.0445) (width 0.254) (layer B.Cu) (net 15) (status 10))
 (segment (start 146.87 39.46) (end 148.14 38.19) (width 0.254) (layer B.Cu) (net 6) (status 20))
 (segment (start 146.87 58.235) (end 146.87 39.46) (width 0.254) (layer B.Cu) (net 6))
 (segment (start 142.875 62.23) (end 146.87 58.235) (width 0.254) (layer B.Cu) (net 6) (status 10))
 (segment (start 146.7389 37.0511) (end 145.6 38.19) (width 0.254) (layer F.Cu) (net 7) (status 20))
 (segment (start 160.9211 37.0511) (end 146.7389 37.0511) (width 0.254) (layer F.Cu) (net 7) (status 10))
 (segment (start 161.23 37.36) (end 160.9211 37.0511) (width 0.254) (layer F.Cu) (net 7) (status 30))
 (segment (start 136.71 44.54) (end 143.06 38.19) (width 0.254) (layer B.Cu) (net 8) (status 20))
 (segment (start 136.71 53.155) (end 136.71 44.54) (width 0.254) (layer B.Cu) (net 8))
 (segment (start 127.635 62.23) (end 136.71 53.155) (width 0.254) (layer B.Cu) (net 8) (status 10))
 (segment (start 163.77 57.75) (end 163.77 55.25) (width 0.254) (layer B.Cu) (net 16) (status 10))
 (segment (start 165.4229 53.3471) (end 163.77 55.25) (width 0.254) (layer B.Cu) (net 16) (status 20))
 (segment (start 165.4229 39.9161) (end 165.4229 53.3471) (width 0.254) (layer B.Cu) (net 16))
 (segment (start 164.1368 38.63) (end 165.4229 39.9161) (width 0.254) (layer B.Cu) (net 16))
 (segment (start 163.424 38.63) (end 164.1368 38.63) (width 0.254) (layer B.Cu) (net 16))
 (segment (start 162.6386 37.8446) (end 163.424 38.63) (width 0.254) (layer B.Cu) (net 16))
 (segment (start 162.6386 37.1037) (end 162.6386 37.8446) (width 0.254) (layer B.Cu) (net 16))
 (segment (start 156.6847 31.1498) (end 162.6386 37.1037) (width 0.254) (layer B.Cu) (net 16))
 (segment (start 131.22 31.1498) (end 156.6847 31.1498) (width 0.254) (layer B.Cu) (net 16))
 (segment (start 127.8698 34.5) (end 131.22 31.1498) (width 0.254) (layer B.Cu) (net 16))
 (segment (start 126.79 34.5) (end 127.8698 34.5) (width 0.254) (layer B.Cu) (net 16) (status 10))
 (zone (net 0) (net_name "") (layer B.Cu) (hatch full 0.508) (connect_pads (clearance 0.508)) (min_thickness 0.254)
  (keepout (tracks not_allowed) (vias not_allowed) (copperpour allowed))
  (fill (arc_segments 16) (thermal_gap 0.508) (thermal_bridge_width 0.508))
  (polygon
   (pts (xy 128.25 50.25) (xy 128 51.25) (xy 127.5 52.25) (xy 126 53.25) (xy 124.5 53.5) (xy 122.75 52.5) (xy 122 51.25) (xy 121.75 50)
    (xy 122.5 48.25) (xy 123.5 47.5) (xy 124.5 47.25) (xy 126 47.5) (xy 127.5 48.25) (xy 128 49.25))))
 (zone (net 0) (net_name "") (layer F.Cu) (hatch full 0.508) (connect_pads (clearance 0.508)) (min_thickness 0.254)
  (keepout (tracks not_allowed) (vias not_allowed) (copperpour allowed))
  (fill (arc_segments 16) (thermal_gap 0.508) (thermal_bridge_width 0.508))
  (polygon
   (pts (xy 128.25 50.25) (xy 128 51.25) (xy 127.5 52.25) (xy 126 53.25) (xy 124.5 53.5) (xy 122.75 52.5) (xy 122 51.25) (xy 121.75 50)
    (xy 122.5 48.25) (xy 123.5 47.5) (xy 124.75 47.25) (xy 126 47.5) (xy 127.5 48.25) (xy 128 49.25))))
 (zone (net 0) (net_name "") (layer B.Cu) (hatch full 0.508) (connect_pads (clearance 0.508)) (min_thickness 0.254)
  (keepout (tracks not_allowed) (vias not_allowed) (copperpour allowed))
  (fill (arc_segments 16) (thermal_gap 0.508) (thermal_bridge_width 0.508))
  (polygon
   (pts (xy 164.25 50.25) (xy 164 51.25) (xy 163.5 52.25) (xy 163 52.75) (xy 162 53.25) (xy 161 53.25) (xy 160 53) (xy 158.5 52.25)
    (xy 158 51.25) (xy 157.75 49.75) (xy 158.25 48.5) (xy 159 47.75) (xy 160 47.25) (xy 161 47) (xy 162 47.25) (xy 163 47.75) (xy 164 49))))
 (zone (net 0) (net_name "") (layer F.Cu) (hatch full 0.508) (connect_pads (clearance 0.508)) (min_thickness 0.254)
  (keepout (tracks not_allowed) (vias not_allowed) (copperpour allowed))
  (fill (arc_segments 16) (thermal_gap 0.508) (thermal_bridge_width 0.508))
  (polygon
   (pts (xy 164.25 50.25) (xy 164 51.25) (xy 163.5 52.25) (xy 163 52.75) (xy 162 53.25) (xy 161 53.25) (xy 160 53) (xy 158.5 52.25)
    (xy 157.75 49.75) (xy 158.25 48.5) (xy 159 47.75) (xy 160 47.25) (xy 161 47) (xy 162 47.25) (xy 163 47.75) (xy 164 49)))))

